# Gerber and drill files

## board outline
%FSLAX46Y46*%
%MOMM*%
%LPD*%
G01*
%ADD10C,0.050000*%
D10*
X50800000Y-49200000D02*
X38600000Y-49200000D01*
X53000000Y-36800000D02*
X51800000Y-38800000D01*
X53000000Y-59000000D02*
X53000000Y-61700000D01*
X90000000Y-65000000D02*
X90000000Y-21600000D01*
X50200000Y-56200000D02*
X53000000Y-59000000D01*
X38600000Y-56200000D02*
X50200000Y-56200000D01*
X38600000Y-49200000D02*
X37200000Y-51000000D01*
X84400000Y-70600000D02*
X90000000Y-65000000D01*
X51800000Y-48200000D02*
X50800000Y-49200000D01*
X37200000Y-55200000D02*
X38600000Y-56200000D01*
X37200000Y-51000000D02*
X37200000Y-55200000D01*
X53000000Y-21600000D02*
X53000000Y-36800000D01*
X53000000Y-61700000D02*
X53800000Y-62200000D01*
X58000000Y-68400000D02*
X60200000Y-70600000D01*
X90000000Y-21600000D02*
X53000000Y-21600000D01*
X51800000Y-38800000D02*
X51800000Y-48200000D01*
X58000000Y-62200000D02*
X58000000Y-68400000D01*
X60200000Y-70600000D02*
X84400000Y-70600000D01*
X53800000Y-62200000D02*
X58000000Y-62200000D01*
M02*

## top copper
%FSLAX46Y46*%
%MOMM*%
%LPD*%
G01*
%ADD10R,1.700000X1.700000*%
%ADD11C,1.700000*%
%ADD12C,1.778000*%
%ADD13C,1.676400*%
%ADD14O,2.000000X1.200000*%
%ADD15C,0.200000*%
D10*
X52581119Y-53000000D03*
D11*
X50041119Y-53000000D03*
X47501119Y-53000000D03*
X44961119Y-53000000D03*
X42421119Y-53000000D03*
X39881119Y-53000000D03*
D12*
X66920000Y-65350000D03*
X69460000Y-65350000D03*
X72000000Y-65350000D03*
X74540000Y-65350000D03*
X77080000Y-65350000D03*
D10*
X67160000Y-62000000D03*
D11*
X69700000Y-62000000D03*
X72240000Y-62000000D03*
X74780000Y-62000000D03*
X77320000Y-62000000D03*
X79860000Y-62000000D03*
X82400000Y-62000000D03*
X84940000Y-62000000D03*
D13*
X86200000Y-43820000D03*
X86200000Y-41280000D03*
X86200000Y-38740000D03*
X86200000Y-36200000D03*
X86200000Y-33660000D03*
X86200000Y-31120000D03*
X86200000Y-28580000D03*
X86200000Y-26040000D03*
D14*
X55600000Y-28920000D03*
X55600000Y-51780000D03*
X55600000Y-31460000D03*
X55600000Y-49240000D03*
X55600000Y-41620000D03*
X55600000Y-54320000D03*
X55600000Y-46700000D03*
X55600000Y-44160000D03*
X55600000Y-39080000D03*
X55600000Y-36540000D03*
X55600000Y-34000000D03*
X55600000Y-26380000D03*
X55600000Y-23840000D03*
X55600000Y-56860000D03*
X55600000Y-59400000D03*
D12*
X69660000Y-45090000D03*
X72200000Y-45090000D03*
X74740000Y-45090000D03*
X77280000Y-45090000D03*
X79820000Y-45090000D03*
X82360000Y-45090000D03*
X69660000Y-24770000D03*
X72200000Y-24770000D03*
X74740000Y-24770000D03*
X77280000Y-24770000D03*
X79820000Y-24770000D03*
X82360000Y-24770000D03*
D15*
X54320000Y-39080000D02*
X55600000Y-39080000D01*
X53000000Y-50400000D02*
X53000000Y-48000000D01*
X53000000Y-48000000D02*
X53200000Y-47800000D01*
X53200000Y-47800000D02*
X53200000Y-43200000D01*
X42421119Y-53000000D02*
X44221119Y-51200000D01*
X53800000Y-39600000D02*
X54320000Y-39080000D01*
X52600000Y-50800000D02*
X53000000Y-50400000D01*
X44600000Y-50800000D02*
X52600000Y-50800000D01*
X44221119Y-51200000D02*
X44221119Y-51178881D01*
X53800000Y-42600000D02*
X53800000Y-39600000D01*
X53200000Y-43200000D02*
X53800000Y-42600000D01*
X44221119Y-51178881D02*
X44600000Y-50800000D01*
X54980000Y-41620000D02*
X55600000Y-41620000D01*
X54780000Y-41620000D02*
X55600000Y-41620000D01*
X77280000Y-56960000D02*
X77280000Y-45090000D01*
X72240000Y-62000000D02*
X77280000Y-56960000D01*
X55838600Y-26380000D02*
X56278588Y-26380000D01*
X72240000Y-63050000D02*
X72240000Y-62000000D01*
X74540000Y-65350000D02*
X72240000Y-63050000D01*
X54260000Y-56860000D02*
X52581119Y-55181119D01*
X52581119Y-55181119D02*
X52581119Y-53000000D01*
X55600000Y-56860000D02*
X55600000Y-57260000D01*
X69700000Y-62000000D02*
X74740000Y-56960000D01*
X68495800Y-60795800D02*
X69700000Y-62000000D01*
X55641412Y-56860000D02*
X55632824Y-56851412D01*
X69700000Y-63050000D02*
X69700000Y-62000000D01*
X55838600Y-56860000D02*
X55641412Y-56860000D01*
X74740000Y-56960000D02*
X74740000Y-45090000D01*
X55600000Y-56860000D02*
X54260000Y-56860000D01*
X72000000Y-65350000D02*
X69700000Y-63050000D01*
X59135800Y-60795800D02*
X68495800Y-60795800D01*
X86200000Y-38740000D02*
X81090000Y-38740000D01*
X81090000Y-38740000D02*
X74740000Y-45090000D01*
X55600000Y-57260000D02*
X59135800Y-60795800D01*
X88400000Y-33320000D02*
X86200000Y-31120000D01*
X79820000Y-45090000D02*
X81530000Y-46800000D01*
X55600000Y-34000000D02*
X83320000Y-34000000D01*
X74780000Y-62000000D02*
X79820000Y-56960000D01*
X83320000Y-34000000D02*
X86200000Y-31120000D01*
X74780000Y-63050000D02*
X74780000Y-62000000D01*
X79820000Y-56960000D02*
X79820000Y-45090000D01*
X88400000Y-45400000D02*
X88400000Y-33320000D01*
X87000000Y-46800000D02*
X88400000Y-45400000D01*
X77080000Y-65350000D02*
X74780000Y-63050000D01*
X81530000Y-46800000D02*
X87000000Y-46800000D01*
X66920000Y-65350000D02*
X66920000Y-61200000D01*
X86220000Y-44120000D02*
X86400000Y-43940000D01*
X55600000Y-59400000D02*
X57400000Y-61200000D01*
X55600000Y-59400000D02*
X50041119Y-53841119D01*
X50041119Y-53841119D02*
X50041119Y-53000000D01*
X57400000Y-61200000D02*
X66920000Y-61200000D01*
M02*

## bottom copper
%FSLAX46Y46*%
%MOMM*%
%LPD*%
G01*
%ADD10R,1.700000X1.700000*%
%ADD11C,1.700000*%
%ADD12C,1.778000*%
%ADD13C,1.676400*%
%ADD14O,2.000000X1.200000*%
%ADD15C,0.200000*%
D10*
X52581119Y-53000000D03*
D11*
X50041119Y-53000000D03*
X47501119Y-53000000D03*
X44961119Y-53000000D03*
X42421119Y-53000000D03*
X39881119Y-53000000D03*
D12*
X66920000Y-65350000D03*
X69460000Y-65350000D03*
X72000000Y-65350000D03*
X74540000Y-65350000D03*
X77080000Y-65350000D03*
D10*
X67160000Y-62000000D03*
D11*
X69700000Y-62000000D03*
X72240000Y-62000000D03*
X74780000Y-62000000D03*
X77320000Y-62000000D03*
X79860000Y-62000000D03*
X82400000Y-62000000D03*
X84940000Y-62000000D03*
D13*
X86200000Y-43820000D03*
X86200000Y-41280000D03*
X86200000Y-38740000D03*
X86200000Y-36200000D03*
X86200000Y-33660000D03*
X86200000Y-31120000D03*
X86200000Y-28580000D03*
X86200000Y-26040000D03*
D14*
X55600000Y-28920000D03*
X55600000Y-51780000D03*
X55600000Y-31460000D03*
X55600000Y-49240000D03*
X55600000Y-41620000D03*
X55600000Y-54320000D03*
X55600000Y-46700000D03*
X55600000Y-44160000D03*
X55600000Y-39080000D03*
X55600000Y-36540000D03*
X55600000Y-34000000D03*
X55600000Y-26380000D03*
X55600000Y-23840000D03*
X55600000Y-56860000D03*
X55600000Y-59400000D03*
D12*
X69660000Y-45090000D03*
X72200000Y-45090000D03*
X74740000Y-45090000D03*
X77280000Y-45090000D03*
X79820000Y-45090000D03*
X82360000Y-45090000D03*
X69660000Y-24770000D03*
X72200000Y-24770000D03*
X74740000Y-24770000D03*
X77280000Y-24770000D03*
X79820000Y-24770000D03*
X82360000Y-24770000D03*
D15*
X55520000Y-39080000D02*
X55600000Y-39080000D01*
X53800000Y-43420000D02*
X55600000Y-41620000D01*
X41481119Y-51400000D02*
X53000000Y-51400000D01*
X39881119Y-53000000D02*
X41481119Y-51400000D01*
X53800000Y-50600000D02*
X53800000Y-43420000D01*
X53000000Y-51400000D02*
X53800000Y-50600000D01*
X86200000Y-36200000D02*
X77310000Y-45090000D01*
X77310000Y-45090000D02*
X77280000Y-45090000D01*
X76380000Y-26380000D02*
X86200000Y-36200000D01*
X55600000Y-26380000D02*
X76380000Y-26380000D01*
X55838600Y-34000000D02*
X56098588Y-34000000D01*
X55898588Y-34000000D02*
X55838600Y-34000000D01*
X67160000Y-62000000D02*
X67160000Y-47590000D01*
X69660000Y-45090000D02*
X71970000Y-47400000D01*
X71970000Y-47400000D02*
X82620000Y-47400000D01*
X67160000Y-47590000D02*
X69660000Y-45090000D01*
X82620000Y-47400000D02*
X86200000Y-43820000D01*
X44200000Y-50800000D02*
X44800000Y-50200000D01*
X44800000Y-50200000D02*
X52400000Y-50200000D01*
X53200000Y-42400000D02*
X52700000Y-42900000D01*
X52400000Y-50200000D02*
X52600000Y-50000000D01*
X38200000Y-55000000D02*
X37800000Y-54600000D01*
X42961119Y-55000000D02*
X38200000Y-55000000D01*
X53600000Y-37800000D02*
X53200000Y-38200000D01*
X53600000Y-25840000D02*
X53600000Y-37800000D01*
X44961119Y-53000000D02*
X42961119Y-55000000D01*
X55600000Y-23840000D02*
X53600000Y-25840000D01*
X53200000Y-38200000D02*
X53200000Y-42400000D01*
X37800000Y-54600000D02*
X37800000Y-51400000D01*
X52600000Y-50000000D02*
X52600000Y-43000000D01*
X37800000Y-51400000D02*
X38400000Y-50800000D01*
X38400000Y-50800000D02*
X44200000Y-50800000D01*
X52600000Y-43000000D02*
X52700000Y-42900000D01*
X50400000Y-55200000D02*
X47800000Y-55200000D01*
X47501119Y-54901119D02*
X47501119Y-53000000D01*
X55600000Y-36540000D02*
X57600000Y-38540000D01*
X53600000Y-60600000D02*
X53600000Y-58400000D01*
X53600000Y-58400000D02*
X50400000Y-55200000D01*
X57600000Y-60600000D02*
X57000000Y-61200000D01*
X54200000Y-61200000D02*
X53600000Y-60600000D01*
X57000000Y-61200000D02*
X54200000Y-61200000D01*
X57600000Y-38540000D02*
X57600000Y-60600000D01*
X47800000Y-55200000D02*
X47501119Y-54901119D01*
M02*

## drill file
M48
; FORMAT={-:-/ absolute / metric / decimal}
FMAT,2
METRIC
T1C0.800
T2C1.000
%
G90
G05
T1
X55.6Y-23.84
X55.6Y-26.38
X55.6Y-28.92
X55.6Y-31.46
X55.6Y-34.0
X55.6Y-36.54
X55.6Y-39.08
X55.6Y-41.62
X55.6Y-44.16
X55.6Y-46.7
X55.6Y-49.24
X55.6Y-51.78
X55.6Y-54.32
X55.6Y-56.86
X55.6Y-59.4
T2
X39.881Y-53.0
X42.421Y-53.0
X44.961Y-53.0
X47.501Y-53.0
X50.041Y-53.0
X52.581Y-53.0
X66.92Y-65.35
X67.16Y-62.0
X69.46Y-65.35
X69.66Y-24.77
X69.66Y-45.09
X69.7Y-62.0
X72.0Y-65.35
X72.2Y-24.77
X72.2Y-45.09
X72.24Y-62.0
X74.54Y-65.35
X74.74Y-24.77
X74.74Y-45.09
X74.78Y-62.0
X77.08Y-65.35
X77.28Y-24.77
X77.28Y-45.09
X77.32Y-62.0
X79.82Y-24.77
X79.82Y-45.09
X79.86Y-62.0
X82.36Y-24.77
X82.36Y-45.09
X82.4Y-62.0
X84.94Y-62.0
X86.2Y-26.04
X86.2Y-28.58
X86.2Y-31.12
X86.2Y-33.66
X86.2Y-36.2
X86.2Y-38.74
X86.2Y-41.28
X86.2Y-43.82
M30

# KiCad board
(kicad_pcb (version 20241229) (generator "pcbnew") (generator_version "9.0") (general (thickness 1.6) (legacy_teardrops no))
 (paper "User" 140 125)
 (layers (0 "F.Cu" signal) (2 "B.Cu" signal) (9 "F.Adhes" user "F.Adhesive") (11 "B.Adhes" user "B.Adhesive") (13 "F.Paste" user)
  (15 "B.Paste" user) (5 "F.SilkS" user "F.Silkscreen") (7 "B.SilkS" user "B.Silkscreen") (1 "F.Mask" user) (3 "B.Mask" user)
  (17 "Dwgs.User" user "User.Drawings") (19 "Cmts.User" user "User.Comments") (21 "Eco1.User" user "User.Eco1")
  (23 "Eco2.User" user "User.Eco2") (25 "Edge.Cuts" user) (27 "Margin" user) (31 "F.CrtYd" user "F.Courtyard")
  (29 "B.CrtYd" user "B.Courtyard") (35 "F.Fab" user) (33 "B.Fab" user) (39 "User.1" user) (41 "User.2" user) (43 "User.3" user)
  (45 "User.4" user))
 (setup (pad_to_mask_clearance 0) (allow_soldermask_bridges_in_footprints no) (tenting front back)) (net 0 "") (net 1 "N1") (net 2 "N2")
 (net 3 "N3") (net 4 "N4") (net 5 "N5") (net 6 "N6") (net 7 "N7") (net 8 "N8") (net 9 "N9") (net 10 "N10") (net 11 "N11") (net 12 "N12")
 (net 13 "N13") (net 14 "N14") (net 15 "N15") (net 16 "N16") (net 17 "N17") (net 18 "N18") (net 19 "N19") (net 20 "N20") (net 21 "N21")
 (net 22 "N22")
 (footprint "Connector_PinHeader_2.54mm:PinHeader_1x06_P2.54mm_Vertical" (layer "F.Cu") (at 52.581119 53 -90)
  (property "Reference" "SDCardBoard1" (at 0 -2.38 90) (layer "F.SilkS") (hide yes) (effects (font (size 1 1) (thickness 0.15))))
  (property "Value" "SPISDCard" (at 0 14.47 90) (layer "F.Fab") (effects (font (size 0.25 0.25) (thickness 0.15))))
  (pad "1" thru_hole rect (at 0 0 270) (size 1.7 1.7) (drill 1) (layers "*.Cu" "*.Mask") (remove_unused_layers no) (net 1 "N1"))
  (pad "2" thru_hole circle (at 0 2.54 270) (size 1.7 1.7) (drill 1) (layers "*.Cu" "*.Mask") (remove_unused_layers no) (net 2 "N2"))
  (pad "3" thru_hole circle (at 0 5.08 270) (size 1.7 1.7) (drill 1) (layers "*.Cu" "*.Mask") (remove_unused_layers no) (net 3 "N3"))
  (pad "4" thru_hole circle (at 0 7.62 270) (size 1.7 1.7) (drill 1) (layers "*.Cu" "*.Mask") (remove_unused_layers no) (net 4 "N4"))
  (pad "5" thru_hole circle (at 0 10.16 270) (size 1.7 1.7) (drill 1) (layers "*.Cu" "*.Mask") (remove_unused_layers no) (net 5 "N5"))
  (pad "6" thru_hole circle (at 0 12.7 270) (size 1.7 1.7) (drill 1) (layers "*.Cu" "*.Mask") (remove_unused_layers no) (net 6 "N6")))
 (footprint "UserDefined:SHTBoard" (layer "F.Cu") (at 72.04 58.699)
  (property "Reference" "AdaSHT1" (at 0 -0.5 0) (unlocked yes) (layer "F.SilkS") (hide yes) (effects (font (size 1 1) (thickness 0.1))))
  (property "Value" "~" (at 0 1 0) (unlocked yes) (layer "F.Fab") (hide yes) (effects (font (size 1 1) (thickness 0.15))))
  (pad "1" thru_hole circle (at -5.12 6.651 90) (size 1.778 1.778) (drill 1) (layers "*.Cu" "*.Mask") (remove_unused_layers no) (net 2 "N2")
   (solder_mask_margin 0.0508) (thermal_bridge_angle 0))
  (pad "2" thru_hole circle (at -2.58 6.651 90) (size 1.778 1.778) (drill 1) (layers "*.Cu" "*.Mask") (remove_unused_layers no) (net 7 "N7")
   (solder_mask_margin 0.0508) (thermal_bridge_angle 0))
  (pad "3" thru_hole circle (at -0.04 6.651 90) (size 1.778 1.778) (drill 1) (layers "*.Cu" "*.Mask") (remove_unused_layers no) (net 1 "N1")
   (solder_mask_margin 0.0508) (thermal_bridge_angle 0))
  (pad "4" thru_hole circle (at 2.5 6.651 90) (size 1.778 1.778) (drill 1) (layers "*.Cu" "*.Mask") (remove_unused_layers no) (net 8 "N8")
   (solder_mask_margin 0.0508) (thermal_bridge_angle 0))
  (pad "5" thru_hole circle (at 5.04 6.651 90) (size 1.778 1.778) (drill 1) (layers "*.Cu" "*.Mask") (remove_unused_layers no) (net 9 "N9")
   (solder_mask_margin 0.0508) (thermal_bridge_angle 0)))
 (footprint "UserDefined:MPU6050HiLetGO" (layer "F.Cu") (at 65.66 64 90)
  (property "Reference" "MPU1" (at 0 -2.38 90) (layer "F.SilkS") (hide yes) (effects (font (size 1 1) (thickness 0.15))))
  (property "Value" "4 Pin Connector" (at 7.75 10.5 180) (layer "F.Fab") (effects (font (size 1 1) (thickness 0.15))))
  (pad "1" thru_hole rect (at 2 1.5 90) (size 1.7 1.7) (drill 1) (layers "*.Cu" "*.Mask") (remove_unused_layers no) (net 2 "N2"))
  (pad "2" thru_hole circle (at 2 4.04 90) (size 1.7 1.7) (drill 1) (layers "*.Cu" "*.Mask") (remove_unused_layers no) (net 1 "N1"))
  (pad "3" thru_hole circle (at 2 6.58 90) (size 1.7 1.7) (drill 1) (layers "*.Cu" "*.Mask") (remove_unused_layers no) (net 8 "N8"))
  (pad "4" thru_hole circle (at 2 9.12 90) (size 1.7 1.7) (drill 1) (layers "*.Cu" "*.Mask") (remove_unused_layers no) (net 9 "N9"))
  (pad "5" thru_hole circle (at 2 11.66 90) (size 1.7 1.7) (drill 1) (layers "*.Cu" "*.Mask") (remove_unused_layers no))
  (pad "6" thru_hole circle (at 2 14.2 90) (size 1.7 1.7) (drill 1) (layers "*.Cu" "*.Mask") (remove_unused_layers no))
  (pad "7" thru_hole circle (at 2 16.74 90) (size 1.7 1.7) (drill 1) (layers "*.Cu" "*.Mask") (remove_unused_layers no))
  (pad "8" thru_hole circle (at 2 19.28 90) (size 1.7 1.7) (drill 1) (layers "*.Cu" "*.Mask") (remove_unused_layers no)))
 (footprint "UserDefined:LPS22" (layer "F.Cu") (at 77.996051 34.473949 90)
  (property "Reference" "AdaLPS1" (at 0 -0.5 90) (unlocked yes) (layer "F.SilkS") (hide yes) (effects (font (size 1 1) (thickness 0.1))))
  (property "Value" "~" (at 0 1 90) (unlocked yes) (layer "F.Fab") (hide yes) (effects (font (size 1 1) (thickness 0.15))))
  (pad "1" thru_hole circle (at -9.346051 8.203949 180) (size 1.6764 1.6764) (drill 1) (layers "*.Cu" "*.Mask") (remove_unused_layers no)
   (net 2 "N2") (solder_mask_margin 0.0508) (thermal_bridge_angle 0))
  (pad "2" thru_hole circle (at -6.806051 8.203949 180) (size 1.6764 1.6764) (drill 1) (layers "*.Cu" "*.Mask") (remove_unused_layers no)
   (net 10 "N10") (solder_mask_margin 0.0508) (thermal_bridge_angle 0))
  (pad "3" thru_hole circle (at -4.266051 8.203949 180) (size 1.6764 1.6764) (drill 1) (layers "*.Cu" "*.Mask") (remove_unused_layers no)
   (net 1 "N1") (solder_mask_margin 0.0508) (thermal_bridge_angle 0))
  (pad "4" thru_hole circle (at -1.726051 8.203949 180) (size 1.6764 1.6764) (drill 1) (layers "*.Cu" "*.Mask") (remove_unused_layers no)
   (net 8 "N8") (solder_mask_margin 0.0508) (thermal_bridge_angle 0))
  (pad "5" thru_hole circle (at 0.813949 8.203949 180) (size 1.6764 1.6764) (drill 1) (layers "*.Cu" "*.Mask") (remove_unused_layers no)
   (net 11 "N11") (solder_mask_margin 0.0508) (thermal_bridge_angle 0))
  (pad "6" thru_hole circle (at 3.353949 8.203949 180) (size 1.6764 1.6764) (drill 1) (layers "*.Cu" "*.Mask") (remove_unused_layers no)
   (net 9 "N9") (solder_mask_margin 0.0508) (thermal_bridge_angle 0))
  (pad "7" thru_hole circle (at 5.893949 8.203949 180) (size 1.6764 1.6764) (drill 1) (layers "*.Cu" "*.Mask") (remove_unused_layers no)
   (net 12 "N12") (solder_mask_margin 0.0508) (thermal_bridge_angle 0))
  (pad "8" thru_hole circle (at 8.433949 8.203949 180) (size 1.6764 1.6764) (drill 1) (layers "*.Cu" "*.Mask") (remove_unused_layers no)
   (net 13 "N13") (solder_mask_margin 0.0508) (thermal_bridge_angle 0)))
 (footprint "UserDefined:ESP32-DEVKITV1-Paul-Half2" (layer "F.Cu") (at 54.1 22.66)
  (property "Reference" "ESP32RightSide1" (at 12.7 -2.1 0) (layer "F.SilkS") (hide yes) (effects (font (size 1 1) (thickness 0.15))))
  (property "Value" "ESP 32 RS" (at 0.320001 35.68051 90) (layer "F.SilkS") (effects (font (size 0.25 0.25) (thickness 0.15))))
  (pad "1" thru_hole oval (at 1.5 6.26 270) (size 1.2 2) (drill 0.8) (layers "*.Cu" "*.Mask") (remove_unused_layers no) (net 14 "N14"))
  (pad "2" thru_hole oval (at 1.5 29.12 270) (size 1.2 2) (drill 0.8) (layers "*.Cu" "*.Mask") (remove_unused_layers no) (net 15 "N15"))
  (pad "3" thru_hole oval (at 1.5 8.8 270) (size 1.2 2) (drill 0.8) (layers "*.Cu" "*.Mask") (remove_unused_layers no) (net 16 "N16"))
  (pad "4" thru_hole oval (at 1.5 26.58 270) (size 1.2 2) (drill 0.8) (layers "*.Cu" "*.Mask") (remove_unused_layers no) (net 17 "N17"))
  (pad "5" thru_hole oval (at 1.5 18.96 270) (size 1.2 2) (drill 0.8) (layers "*.Cu" "*.Mask") (remove_unused_layers no) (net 6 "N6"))
  (pad "15" thru_hole oval (at 1.5 31.66 270) (size 1.2 2) (drill 0.8) (layers "*.Cu" "*.Mask") (remove_unused_layers no) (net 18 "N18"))
  (pad "16" thru_hole oval (at 1.5 24.04 270) (size 1.2 2) (drill 0.8) (layers "*.Cu" "*.Mask") (remove_unused_layers no) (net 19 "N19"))
  (pad "17" thru_hole oval (at 1.5 21.5 270) (size 1.2 2) (drill 0.8) (layers "*.Cu" "*.Mask") (remove_unused_layers no) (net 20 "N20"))
  (pad "18" thru_hole oval (at 1.5 16.42 270) (size 1.2 2) (drill 0.8) (layers "*.Cu" "*.Mask") (remove_unused_layers no) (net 5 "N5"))
  (pad "19" thru_hole oval (at 1.5 13.88 270) (size 1.2 2) (drill 0.8) (layers "*.Cu" "*.Mask") (remove_unused_layers no) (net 3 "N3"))
  (pad "21" thru_hole oval (at 1.5 11.34 270) (size 1.2 2) (drill 0.8) (layers "*.Cu" "*.Mask") (remove_unused_layers no) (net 9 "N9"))
  (pad "22" thru_hole oval (at 1.5 3.72 270) (size 1.2 2) (drill 0.8) (layers "*.Cu" "*.Mask") (remove_unused_layers no) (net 8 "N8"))
  (pad "23" thru_hole oval (at 1.5 1.18 270) (size 1.2 2) (drill 0.8) (layers "*.Cu" "*.Mask") (remove_unused_layers no) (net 4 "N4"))
  (pad "53" thru_hole oval (at 1.5 34.2 270) (size 1.2 2) (drill 0.8) (layers "*.Cu" "*.Mask") (remove_unused_layers no) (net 1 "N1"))
  (pad "54" thru_hole oval (at 1.5 36.74 270) (size 1.2 2) (drill 0.8) (layers "*.Cu" "*.Mask") (remove_unused_layers no) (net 2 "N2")))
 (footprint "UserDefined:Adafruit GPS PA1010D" (layer "F.Cu") (at 83.053949 39.886051)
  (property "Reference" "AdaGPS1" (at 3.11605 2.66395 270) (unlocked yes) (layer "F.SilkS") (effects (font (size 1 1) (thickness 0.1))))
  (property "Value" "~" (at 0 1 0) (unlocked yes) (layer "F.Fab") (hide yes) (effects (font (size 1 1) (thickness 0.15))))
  (pad "1" thru_hole circle (at -13.393949 5.203949 90) (size 1.778 1.778) (drill 1) (layers "*.Cu" "*.Mask") (remove_unused_layers no)
   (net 2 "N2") (solder_mask_margin 0.0508) (thermal_bridge_angle 0))
  (pad "2" thru_hole circle (at -10.853949 5.203949 90) (size 1.778 1.778) (drill 1) (layers "*.Cu" "*.Mask") (remove_unused_layers no)
   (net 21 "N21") (solder_mask_margin 0.0508) (thermal_bridge_angle 0))
  (pad "3" thru_hole circle (at -8.313949 5.203949 90) (size 1.778 1.778) (drill 1) (layers "*.Cu" "*.Mask") (remove_unused_layers no)
   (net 1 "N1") (solder_mask_margin 0.0508) (thermal_bridge_angle 0))
  (pad "4" thru_hole circle (at -5.773949 5.203949 90) (size 1.778 1.778) (drill 1) (layers "*.Cu" "*.Mask") (remove_unused_layers no)
   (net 8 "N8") (solder_mask_margin 0.0508) (thermal_bridge_angle 0))
  (pad "5" thru_hole circle (at -3.233949 5.203949 90) (size 1.778 1.778) (drill 1) (layers "*.Cu" "*.Mask") (remove_unused_layers no)
   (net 9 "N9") (solder_mask_margin 0.0508) (thermal_bridge_angle 0))
  (pad "6" thru_hole circle (at -0.693949 5.203949 90) (size 1.778 1.778) (drill 1) (layers "*.Cu" "*.Mask") (remove_unused_layers no)
   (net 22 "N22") (solder_mask_margin 0.0508) (thermal_bridge_angle 0))
  (pad "7" thru_hole circle (at -13.393949 -15.116051 90) (size 1.778 1.778) (drill 1) (layers "*.Cu" "*.Mask") (remove_unused_layers no)
   (solder_mask_margin 0.0508) (thermal_bridge_angle 0))
  (pad "8" thru_hole circle (at -10.853949 -15.116051 90) (size 1.778 1.778) (drill 1) (layers "*.Cu" "*.Mask") (remove_unused_layers no)
   (solder_mask_margin 0.0508) (thermal_bridge_angle 0))
  (pad "9" thru_hole circle (at -8.313949 -15.116051 90) (size 1.778 1.778) (drill 1) (layers "*.Cu" "*.Mask") (remove_unused_layers no)
   (solder_mask_margin 0.0508) (thermal_bridge_angle 0))
  (pad "10" thru_hole circle (at -5.773949 -15.116051 90) (size 1.778 1.778) (drill 1) (layers "*.Cu" "*.Mask") (remove_unused_layers no)
   (solder_mask_margin 0.0508) (thermal_bridge_angle 0))
  (pad "11" thru_hole circle (at -3.233949 -15.116051 90) (size 1.778 1.778) (drill 1) (layers "*.Cu" "*.Mask") (remove_unused_layers no)
   (solder_mask_margin 0.0508) (thermal_bridge_angle 0))
  (pad "12" thru_hole circle (at -0.693949 -15.116051 90) (size 1.778 1.778) (drill 1) (layers "*.Cu" "*.Mask") (remove_unused_layers no)
   (solder_mask_margin 0.0508) (thermal_bridge_angle 0)))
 (gr_line (start 50.8 49.2) (end 38.6 49.2) (stroke (width 0.05) (type default)) (layer "Edge.Cuts"))
 (gr_line (start 53 36.8) (end 51.8 38.8) (stroke (width 0.05) (type default)) (layer "Edge.Cuts"))
 (gr_line (start 53 59) (end 53 61.7) (stroke (width 0.05) (type default)) (layer "Edge.Cuts"))
 (gr_line (start 90 65) (end 90 21.6) (stroke (width 0.05) (type default)) (layer "Edge.Cuts"))
 (gr_line (start 50.2 56.2) (end 53 59) (stroke (width 0.05) (type default)) (layer "Edge.Cuts"))
 (gr_line (start 38.6 56.2) (end 50.2 56.2) (stroke (width 0.05) (type default)) (layer "Edge.Cuts"))
 (gr_line (start 38.6 49.2) (end 37.2 51) (stroke (width 0.05) (type default)) (layer "Edge.Cuts"))
 (gr_line (start 84.4 70.6) (end 90 65) (stroke (width 0.05) (type default)) (layer "Edge.Cuts"))
 (gr_line (start 51.8 48.2) (end 50.8 49.2) (stroke (width 0.05) (type default)) (layer "Edge.Cuts"))
 (gr_line (start 37.2 55.2) (end 38.6 56.2) (stroke (width 0.05) (type default)) (layer "Edge.Cuts"))
 (gr_line (start 37.2 51) (end 37.2 55.2) (stroke (width 0.05) (type default)) (layer "Edge.Cuts"))
 (gr_line (start 53 21.6) (end 53 36.8) (stroke (width 0.05) (type default)) (layer "Edge.Cuts"))
 (gr_line (start 53 61.7) (end 53.8 62.2) (stroke (width 0.05) (type default)) (layer "Edge.Cuts"))
 (gr_line (start 58 68.4) (end 60.2 70.6) (stroke (width 0.05) (type default)) (layer "Edge.Cuts"))
 (gr_line (start 90 21.6) (end 53 21.6) (stroke (width 0.05) (type default)) (layer "Edge.Cuts"))
 (gr_line (start 51.8 38.8) (end 51.8 48.2) (stroke (width 0.05) (type default)) (layer "Edge.Cuts"))
 (gr_line (start 58 62.2) (end 58 68.4) (stroke (width 0.05) (type default)) (layer "Edge.Cuts"))
 (gr_line (start 60.2 70.6) (end 84.4 70.6) (stroke (width 0.05) (type default)) (layer "Edge.Cuts"))
 (gr_line (start 53.8 62.2) (end 58 62.2) (stroke (width 0.05) (type default)) (layer "Edge.Cuts"))
 (segment (start 54.32 39.08) (end 55.6 39.08) (width 0.2) (layer "F.Cu") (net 5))
 (segment (start 53 50.4) (end 53 48) (width 0.2) (layer "F.Cu") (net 5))
 (segment (start 53 48) (end 53.2 47.8) (width 0.2) (layer "F.Cu") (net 5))
 (segment (start 53.2 47.8) (end 53.2 43.2) (width 0.2) (layer "F.Cu") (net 5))
 (segment (start 42.421119 53) (end 44.221119 51.2) (width 0.2) (layer "F.Cu") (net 5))
 (segment (start 53.8 39.6) (end 54.32 39.08) (width 0.2) (layer "F.Cu") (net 5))
 (segment (start 52.6 50.8) (end 53 50.4) (width 0.2) (layer "F.Cu") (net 5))
 (segment (start 44.6 50.8) (end 52.6 50.8) (width 0.2) (layer "F.Cu") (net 5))
 (segment (start 44.221119 51.2) (end 44.221119 51.178881) (width 0.2) (layer "F.Cu") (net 5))
 (segment (start 53.8 42.6) (end 53.8 39.6) (width 0.2) (layer "F.Cu") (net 5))
 (segment (start 53.2 43.2) (end 53.8 42.6) (width 0.2) (layer "F.Cu") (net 5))
 (segment (start 44.221119 51.178881) (end 44.6 50.8) (width 0.2) (layer "F.Cu") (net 5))
 (segment (start 55.52 39.08) (end 55.6 39.08) (width 0.2) (layer "B.Cu") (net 5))
 (segment (start 54.98 41.62) (end 55.6 41.62) (width 0.2) (layer "F.Cu") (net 6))
 (segment (start 54.78 41.62) (end 55.6 41.62) (width 0.2) (layer "F.Cu") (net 6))
 (segment (start 53.8 43.42) (end 55.6 41.62) (width 0.2) (layer "B.Cu") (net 6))
 (segment (start 41.481119 51.4) (end 53 51.4) (width 0.2) (layer "B.Cu") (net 6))
 (segment (start 39.881119 53) (end 41.481119 51.4) (width 0.2) (layer "B.Cu") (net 6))
 (segment (start 53.8 50.6) (end 53.8 43.42) (width 0.2) (layer "B.Cu") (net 6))
 (segment (start 53 51.4) (end 53.8 50.6) (width 0.2) (layer "B.Cu") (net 6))
 (segment (start 77.28 56.96) (end 77.28 45.09) (width 0.2) (layer "F.Cu") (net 8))
 (segment (start 72.24 62) (end 77.28 56.96) (width 0.2) (layer "F.Cu") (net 8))
 (segment (start 55.8386 26.38) (end 56.278588 26.38) (width 0.2) (layer "F.Cu") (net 8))
 (segment (start 72.24 63.05) (end 72.24 62) (width 0.2) (layer "F.Cu") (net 8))
 (segment (start 74.54 65.35) (end 72.24 63.05) (width 0.2) (layer "F.Cu") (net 8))
 (segment (start 86.2 36.2) (end 77.31 45.09) (width 0.2) (layer "B.Cu") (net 8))
 (segment (start 77.31 45.09) (end 77.28 45.09) (width 0.2) (layer "B.Cu") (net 8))
 (segment (start 76.38 26.38) (end 86.2 36.2) (width 0.2) (layer "B.Cu") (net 8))
 (segment (start 55.6 26.38) (end 76.38 26.38) (width 0.2) (layer "B.Cu") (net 8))
 (segment (start 54.26 56.86) (end 52.581119 55.181119) (width 0.2) (layer "F.Cu") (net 1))
 (segment (start 52.581119 55.181119) (end 52.581119 53) (width 0.2) (layer "F.Cu") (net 1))
 (segment (start 55.6 56.86) (end 55.6 57.26) (width 0.2) (layer "F.Cu") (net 1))
 (segment (start 69.7 62) (end 74.74 56.96) (width 0.2) (layer "F.Cu") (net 1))
 (segment (start 68.4958 60.7958) (end 69.7 62) (width 0.2) (layer "F.Cu") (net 1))
 (segment (start 55.641412 56.86) (end 55.632824 56.851412) (width 0.2) (layer "F.Cu") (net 1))
 (segment (start 69.7 63.05) (end 69.7 62) (width 0.2) (layer "F.Cu") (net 1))
 (segment (start 55.8386 56.86) (end 55.641412 56.86) (width 0.2) (layer "F.Cu") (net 1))
 (segment (start 74.74 56.96) (end 74.74 45.09) (width 0.2) (layer "F.Cu") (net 1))
 (segment (start 55.6 56.86) (end 54.26 56.86) (width 0.2) (layer "F.Cu") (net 1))
 (segment (start 72 65.35) (end 69.7 63.05) (width 0.2) (layer "F.Cu") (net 1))
 (segment (start 59.1358 60.7958) (end 68.4958 60.7958) (width 0.2) (layer "F.Cu") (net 1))
 (segment (start 86.2 38.74) (end 81.09 38.74) (width 0.2) (layer "F.Cu") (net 1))
 (segment (start 81.09 38.74) (end 74.74 45.09) (width 0.2) (layer "F.Cu") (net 1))
 (segment (start 55.6 57.26) (end 59.1358 60.7958) (width 0.2) (layer "F.Cu") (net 1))
 (segment (start 88.4 33.32) (end 86.2 31.12) (width 0.2) (layer "F.Cu") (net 9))
 (segment (start 79.82 45.09) (end 81.53 46.8) (width 0.2) (layer "F.Cu") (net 9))
 (segment (start 55.6 34) (end 83.32 34) (width 0.2) (layer "F.Cu") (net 9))
 (segment (start 74.78 62) (end 79.82 56.96) (width 0.2) (layer "F.Cu") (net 9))
 (segment (start 83.32 34) (end 86.2 31.12) (width 0.2) (layer "F.Cu") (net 9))
 (segment (start 74.78 63.05) (end 74.78 62) (width 0.2) (layer "F.Cu") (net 9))
 (segment (start 79.82 56.96) (end 79.82 45.09) (width 0.2) (layer "F.Cu") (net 9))
 (segment (start 88.4 45.4) (end 88.4 33.32) (width 0.2) (layer "F.Cu") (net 9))
 (segment (start 87 46.8) (end 88.4 45.4) (width 0.2) (layer "F.Cu") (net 9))
 (segment (start 77.08 65.35) (end 74.78 63.05) (width 0.2) (layer "F.Cu") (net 9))
 (segment (start 81.53 46.8) (end 87 46.8) (width 0.2) (layer "F.Cu") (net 9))
 (segment (start 55.8386 34) (end 56.098588 34) (width 0.2) (layer "B.Cu") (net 9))
 (segment (start 55.898588 34) (end 55.8386 34) (width 0.2) (layer "B.Cu") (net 9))
 (segment (start 66.92 65.35) (end 66.92 61.2) (width 0.2) (layer "F.Cu") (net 2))
 (segment (start 86.22 44.12) (end 86.4 43.94) (width 0.2) (layer "F.Cu") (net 2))
 (segment (start 55.6 59.4) (end 57.4 61.2) (width 0.2) (layer "F.Cu") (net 2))
 (segment (start 55.6 59.4) (end 50.041119 53.841119) (width 0.2) (layer "F.Cu") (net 2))
 (segment (start 50.041119 53.841119) (end 50.041119 53) (width 0.2) (layer "F.Cu") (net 2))
 (segment (start 57.4 61.2) (end 66.92 61.2) (width 0.2) (layer "F.Cu") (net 2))
 (segment (start 67.16 62) (end 67.16 47.59) (width 0.2) (layer "B.Cu") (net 2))
 (segment (start 69.66 45.09) (end 71.97 47.4) (width 0.2) (layer "B.Cu") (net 2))
 (segment (start 71.97 47.4) (end 82.62 47.4) (width 0.2) (layer "B.Cu") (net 2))
 (segment (start 67.16 47.59) (end 69.66 45.09) (width 0.2) (layer "B.Cu") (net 2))
 (segment (start 82.62 47.4) (end 86.2 43.82) (width 0.2) (layer "B.Cu") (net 2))
 (segment (start 44.2 50.8) (end 44.8 50.2) (width 0.2) (layer "B.Cu") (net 4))
 (segment (start 44.8 50.2) (end 52.4 50.2) (width 0.2) (layer "B.Cu") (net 4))
 (segment (start 53.2 42.4) (end 52.7 42.9) (width 0.2) (layer "B.Cu") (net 4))
 (segment (start 52.4 50.2) (end 52.6 50) (width 0.2) (layer "B.Cu") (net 4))
 (segment (start 38.2 55) (end 37.8 54.6) (width 0.2) (layer "B.Cu") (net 4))
 (segment (start 42.961119 55) (end 38.2 55) (width 0.2) (layer "B.Cu") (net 4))
 (segment (start 53.6 37.8) (end 53.2 38.2) (width 0.2) (layer "B.Cu") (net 4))
 (segment (start 53.6 25.84) (end 53.6 37.8) (width 0.2) (layer "B.Cu") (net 4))
 (segment (start 44.961119 53) (end 42.961119 55) (width 0.2) (layer "B.Cu") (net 4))
 (segment (start 55.6 23.84) (end 53.6 25.84) (width 0.2) (layer "B.Cu") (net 4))
 (segment (start 53.2 38.2) (end 53.2 42.4) (width 0.2) (layer "B.Cu") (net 4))
 (segment (start 37.8 54.6) (end 37.8 51.4) (width 0.2) (layer "B.Cu") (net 4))
 (segment (start 52.6 50) (end 52.6 43) (width 0.2) (layer "B.Cu") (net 4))
 (segment (start 37.8 51.4) (end 38.4 50.8) (width 0.2) (layer "B.Cu") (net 4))
 (segment (start 38.4 50.8) (end 44.2 50.8) (width 0.2) (layer "B.Cu") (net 4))
 (segment (start 52.6 43) (end 52.7 42.9) (width 0.2) (layer "B.Cu") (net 4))
 (segment (start 50.4 55.2) (end 47.8 55.2) (width 0.2) (layer "B.Cu") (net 3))
 (segment (start 47.501119 54.901119) (end 47.501119 53) (width 0.2) (layer "B.Cu") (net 3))
 (segment (start 55.6 36.54) (end 57.6 38.54) (width 0.2) (layer "B.Cu") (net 3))
 (segment (start 53.6 60.6) (end 53.6 58.4) (width 0.2) (layer "B.Cu") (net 3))
 (segment (start 53.6 58.4) (end 50.4 55.2) (width 0.2) (layer "B.Cu") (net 3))
 (segment (start 57.6 60.6) (end 57 61.2) (width 0.2) (layer "B.Cu") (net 3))
 (segment (start 54.2 61.2) (end 53.6 60.6) (width 0.2) (layer "B.Cu") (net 3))
 (segment (start 57 61.2) (end 54.2 61.2) (width 0.2) (layer "B.Cu") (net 3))
 (segment (start 57.6 38.54) (end 57.6 60.6) (width 0.2) (layer "B.Cu") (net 3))
 (segment (start 47.8 55.2) (end 47.501119 54.901119) (width 0.2) (layer "B.Cu") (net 3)))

